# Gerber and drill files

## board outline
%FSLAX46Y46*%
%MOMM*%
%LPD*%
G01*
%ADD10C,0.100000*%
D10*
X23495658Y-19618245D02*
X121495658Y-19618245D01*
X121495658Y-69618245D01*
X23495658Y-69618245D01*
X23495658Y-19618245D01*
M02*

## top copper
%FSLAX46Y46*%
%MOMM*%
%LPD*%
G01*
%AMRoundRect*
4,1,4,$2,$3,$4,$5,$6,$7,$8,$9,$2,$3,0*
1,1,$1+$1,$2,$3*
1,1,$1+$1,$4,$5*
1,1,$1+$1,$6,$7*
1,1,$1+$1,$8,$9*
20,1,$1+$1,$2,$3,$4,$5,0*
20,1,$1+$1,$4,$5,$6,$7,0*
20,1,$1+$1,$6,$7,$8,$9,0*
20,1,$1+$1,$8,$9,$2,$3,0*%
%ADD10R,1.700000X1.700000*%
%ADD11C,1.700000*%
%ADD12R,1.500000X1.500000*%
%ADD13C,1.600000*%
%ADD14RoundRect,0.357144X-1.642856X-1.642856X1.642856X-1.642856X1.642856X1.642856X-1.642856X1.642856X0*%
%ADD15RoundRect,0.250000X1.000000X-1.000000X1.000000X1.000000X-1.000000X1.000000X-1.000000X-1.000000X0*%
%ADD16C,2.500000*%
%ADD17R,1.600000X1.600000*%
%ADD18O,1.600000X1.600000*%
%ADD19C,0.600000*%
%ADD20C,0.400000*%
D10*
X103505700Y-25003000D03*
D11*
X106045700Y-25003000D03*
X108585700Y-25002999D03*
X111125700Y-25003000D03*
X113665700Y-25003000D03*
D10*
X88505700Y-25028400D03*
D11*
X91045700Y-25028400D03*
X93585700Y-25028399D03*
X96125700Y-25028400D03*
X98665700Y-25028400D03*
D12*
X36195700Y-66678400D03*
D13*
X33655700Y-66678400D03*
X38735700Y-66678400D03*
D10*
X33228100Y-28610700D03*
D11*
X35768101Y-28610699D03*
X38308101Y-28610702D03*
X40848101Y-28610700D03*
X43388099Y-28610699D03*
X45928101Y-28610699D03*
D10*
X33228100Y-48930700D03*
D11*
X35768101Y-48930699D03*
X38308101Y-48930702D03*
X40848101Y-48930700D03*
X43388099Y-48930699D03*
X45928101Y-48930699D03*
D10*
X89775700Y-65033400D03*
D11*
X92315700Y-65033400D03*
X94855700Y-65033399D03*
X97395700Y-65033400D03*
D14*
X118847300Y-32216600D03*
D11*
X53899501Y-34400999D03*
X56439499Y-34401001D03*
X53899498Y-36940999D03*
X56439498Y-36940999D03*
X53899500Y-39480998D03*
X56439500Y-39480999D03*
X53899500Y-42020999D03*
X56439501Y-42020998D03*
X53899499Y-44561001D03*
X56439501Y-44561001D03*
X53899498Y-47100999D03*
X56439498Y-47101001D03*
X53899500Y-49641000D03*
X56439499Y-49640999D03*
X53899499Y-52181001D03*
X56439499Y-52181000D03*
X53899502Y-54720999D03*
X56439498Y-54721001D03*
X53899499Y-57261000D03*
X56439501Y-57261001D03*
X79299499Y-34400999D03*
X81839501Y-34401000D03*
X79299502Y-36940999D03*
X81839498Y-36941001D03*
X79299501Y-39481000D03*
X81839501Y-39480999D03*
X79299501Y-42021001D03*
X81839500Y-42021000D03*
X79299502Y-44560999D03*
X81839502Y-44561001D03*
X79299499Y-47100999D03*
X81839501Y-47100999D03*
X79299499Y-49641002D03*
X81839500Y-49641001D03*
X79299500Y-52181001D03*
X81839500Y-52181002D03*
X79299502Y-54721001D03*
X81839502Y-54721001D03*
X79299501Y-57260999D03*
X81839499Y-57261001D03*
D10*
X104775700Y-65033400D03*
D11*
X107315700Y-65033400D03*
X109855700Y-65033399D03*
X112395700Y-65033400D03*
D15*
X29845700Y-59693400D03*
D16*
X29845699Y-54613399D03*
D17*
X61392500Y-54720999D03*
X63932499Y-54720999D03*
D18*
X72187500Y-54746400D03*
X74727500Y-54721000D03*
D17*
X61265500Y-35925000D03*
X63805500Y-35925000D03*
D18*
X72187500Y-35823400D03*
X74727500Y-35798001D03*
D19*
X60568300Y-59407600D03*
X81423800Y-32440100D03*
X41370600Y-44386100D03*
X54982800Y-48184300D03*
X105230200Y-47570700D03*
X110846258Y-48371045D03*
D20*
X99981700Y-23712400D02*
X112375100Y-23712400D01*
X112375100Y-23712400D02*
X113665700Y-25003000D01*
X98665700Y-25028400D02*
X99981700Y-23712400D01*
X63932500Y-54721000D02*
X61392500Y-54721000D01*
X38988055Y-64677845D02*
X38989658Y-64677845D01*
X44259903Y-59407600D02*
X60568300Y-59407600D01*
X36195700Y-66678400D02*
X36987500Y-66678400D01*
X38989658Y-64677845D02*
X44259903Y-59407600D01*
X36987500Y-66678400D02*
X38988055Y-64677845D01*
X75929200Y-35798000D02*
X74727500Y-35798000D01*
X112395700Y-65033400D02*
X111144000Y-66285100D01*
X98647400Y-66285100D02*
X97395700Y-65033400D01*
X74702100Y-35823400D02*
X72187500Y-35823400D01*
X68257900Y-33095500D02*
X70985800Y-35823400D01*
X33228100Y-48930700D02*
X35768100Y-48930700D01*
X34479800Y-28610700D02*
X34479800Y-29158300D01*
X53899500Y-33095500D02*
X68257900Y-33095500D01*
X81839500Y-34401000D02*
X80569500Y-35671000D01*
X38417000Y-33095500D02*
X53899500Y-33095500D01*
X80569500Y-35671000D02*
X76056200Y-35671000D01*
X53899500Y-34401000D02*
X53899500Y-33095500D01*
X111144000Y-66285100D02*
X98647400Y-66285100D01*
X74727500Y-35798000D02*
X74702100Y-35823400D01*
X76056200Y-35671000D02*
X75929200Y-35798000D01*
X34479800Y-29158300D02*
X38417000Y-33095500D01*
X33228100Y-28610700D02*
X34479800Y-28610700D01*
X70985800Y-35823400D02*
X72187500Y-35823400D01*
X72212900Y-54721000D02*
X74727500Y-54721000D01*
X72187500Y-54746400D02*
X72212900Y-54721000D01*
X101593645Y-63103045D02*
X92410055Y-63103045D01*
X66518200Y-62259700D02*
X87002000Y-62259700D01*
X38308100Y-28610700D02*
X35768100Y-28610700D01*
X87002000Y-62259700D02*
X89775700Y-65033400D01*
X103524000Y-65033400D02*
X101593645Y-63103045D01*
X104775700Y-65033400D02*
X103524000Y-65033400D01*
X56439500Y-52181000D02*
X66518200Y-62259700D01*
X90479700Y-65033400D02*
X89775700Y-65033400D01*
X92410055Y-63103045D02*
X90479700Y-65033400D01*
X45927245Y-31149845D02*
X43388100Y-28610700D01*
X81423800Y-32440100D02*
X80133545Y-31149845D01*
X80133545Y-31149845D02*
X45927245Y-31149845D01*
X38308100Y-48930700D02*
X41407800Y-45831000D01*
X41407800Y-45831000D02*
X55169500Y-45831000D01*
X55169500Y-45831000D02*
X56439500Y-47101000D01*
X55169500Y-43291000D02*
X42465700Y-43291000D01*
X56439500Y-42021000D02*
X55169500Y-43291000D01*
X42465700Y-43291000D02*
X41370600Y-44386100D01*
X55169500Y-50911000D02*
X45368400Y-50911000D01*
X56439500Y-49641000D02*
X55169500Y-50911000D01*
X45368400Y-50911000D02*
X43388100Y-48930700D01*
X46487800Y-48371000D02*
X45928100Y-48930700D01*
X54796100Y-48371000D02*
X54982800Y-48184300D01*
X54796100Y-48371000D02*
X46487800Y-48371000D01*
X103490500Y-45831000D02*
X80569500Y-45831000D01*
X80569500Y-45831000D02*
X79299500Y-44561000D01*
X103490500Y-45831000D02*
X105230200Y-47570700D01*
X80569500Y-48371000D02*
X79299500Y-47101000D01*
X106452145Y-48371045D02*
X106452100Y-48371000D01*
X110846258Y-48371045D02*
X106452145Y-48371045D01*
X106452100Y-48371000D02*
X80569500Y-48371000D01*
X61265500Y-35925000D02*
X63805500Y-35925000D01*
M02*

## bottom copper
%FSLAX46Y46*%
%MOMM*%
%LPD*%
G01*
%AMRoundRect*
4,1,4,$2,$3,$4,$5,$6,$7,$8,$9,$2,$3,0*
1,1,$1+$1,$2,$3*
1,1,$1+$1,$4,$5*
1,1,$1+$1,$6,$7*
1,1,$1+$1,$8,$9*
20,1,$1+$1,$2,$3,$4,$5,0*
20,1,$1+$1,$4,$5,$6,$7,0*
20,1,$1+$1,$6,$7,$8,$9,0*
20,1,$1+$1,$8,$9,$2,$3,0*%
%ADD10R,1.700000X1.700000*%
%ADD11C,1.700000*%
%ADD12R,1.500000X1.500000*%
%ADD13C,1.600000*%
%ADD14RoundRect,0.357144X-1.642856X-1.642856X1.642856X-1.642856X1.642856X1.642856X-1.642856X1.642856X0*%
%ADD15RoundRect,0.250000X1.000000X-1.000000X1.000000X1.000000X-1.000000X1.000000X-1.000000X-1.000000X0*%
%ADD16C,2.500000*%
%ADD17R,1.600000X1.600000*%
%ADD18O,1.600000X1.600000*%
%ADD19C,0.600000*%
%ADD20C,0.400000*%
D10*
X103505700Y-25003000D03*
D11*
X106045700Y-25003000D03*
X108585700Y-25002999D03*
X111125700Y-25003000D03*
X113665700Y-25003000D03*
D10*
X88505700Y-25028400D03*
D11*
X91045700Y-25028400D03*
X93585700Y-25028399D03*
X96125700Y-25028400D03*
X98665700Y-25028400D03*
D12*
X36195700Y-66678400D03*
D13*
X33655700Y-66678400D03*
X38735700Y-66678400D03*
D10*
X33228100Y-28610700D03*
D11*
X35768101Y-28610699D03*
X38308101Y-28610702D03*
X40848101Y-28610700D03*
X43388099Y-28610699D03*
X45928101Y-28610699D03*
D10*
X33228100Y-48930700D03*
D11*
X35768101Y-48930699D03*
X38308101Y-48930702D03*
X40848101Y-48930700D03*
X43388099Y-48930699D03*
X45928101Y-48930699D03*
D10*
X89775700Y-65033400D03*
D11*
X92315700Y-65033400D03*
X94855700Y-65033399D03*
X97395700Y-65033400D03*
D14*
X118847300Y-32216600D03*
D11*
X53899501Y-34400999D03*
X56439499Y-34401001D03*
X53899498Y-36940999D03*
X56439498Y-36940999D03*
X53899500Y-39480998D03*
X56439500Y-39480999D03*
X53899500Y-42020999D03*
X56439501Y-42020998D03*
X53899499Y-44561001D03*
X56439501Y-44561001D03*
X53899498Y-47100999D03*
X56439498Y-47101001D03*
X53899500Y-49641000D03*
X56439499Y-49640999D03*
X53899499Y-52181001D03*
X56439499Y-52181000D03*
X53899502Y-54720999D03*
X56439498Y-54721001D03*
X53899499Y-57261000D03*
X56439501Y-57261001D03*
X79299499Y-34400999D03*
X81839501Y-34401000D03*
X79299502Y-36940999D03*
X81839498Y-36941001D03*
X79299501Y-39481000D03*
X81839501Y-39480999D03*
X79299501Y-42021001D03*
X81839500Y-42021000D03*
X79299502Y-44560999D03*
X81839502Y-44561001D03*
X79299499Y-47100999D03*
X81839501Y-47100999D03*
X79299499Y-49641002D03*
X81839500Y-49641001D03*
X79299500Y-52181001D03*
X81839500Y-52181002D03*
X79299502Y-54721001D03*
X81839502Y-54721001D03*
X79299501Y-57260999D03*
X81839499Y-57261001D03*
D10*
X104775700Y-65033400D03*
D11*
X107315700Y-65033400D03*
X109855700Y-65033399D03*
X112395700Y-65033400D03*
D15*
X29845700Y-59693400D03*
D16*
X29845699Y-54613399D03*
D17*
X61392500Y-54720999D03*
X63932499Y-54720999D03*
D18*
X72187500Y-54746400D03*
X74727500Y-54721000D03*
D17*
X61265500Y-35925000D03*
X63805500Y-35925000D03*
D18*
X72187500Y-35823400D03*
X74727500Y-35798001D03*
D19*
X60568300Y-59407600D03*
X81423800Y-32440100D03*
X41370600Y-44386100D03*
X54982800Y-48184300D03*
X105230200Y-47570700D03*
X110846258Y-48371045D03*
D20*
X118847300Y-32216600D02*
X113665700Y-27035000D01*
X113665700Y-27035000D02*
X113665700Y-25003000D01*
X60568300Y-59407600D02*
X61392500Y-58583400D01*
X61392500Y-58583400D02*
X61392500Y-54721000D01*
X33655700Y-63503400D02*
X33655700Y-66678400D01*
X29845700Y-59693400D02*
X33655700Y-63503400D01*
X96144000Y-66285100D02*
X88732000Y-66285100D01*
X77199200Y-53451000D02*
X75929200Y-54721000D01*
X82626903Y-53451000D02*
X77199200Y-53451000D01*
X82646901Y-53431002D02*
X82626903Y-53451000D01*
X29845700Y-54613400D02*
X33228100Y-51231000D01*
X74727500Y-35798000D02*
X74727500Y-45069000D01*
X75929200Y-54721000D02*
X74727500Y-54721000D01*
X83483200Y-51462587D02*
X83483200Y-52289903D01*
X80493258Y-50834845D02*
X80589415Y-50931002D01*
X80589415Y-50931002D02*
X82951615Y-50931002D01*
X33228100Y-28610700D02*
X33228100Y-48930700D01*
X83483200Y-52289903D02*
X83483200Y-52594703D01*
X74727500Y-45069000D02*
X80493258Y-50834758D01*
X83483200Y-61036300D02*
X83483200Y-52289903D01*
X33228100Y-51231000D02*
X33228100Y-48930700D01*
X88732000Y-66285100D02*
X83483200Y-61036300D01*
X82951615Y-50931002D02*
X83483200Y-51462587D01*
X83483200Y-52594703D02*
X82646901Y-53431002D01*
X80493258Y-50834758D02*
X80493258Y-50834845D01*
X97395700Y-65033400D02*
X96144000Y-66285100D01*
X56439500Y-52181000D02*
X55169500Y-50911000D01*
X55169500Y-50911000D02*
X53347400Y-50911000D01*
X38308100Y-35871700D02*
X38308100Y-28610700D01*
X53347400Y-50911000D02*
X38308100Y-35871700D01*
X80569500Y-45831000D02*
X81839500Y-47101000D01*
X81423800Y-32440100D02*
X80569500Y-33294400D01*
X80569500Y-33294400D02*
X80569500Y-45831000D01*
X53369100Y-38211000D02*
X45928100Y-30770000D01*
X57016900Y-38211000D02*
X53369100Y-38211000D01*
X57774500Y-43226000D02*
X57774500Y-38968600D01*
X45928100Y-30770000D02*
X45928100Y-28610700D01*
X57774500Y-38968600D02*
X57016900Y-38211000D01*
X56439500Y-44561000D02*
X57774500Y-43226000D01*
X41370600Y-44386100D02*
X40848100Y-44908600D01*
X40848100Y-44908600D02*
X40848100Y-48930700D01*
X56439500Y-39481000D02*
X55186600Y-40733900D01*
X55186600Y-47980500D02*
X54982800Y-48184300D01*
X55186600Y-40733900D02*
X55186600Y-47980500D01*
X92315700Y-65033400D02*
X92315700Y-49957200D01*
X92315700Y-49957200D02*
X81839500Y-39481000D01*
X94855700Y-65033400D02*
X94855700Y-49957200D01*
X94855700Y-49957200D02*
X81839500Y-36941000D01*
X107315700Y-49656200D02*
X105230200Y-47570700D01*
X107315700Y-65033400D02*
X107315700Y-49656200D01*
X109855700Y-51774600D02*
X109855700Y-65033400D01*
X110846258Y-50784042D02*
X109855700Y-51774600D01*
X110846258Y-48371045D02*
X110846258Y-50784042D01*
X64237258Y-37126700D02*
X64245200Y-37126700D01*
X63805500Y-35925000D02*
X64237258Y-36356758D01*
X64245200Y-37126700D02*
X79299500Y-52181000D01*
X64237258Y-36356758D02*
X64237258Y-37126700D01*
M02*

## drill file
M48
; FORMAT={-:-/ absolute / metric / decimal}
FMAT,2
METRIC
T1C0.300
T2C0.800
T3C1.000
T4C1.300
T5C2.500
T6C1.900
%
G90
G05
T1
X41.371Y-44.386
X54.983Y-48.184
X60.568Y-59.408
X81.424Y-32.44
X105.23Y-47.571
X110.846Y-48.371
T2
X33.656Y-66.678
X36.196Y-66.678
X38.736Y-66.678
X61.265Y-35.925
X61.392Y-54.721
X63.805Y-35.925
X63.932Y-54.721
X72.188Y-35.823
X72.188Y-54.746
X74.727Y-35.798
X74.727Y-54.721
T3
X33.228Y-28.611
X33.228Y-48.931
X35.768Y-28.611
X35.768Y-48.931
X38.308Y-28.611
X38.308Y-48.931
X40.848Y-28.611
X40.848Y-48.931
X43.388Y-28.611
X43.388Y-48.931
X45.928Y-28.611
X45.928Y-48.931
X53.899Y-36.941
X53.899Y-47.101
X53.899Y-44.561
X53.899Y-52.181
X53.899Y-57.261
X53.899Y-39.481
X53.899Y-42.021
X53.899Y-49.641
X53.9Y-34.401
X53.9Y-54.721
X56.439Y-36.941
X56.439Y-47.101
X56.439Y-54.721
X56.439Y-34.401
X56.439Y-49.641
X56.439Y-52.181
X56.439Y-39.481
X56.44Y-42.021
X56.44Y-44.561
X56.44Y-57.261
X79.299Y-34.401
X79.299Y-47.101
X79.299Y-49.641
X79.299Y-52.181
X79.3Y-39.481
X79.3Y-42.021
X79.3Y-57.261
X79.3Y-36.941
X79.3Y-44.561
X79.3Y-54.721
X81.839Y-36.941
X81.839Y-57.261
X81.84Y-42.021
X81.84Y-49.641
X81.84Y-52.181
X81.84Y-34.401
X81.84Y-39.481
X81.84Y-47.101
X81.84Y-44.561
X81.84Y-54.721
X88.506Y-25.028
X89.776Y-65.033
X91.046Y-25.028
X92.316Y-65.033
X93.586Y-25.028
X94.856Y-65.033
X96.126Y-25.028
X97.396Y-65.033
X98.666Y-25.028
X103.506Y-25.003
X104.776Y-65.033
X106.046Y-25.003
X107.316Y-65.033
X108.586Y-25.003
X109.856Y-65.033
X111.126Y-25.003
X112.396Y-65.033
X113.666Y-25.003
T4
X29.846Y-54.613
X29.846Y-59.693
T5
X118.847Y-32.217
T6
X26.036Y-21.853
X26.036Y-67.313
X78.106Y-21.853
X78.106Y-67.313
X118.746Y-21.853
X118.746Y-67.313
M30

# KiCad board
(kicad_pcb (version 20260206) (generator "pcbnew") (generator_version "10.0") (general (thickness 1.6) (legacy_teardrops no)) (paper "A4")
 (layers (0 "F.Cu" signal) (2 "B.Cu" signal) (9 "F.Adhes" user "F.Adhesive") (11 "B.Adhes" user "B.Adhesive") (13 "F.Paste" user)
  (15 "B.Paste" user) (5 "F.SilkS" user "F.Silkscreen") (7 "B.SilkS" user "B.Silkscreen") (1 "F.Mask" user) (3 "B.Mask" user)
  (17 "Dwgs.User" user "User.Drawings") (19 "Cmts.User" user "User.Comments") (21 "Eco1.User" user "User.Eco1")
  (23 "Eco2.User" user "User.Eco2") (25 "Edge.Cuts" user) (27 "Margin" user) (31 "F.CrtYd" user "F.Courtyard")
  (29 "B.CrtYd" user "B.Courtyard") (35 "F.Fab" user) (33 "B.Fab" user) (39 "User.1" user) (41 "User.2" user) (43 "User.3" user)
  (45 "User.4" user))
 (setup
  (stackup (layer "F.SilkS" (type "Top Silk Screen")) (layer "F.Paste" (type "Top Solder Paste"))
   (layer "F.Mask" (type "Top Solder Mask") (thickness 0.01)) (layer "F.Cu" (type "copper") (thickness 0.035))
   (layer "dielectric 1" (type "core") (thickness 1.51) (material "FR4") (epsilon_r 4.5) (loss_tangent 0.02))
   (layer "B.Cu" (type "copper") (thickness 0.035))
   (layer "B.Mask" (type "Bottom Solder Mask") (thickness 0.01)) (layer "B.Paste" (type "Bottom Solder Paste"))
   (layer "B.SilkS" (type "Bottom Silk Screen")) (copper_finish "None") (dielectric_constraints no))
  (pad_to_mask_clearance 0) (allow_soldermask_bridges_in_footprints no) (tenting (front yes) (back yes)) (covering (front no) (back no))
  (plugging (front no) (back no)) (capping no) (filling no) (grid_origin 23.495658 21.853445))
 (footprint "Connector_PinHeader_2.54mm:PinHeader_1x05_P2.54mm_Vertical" (layer "F.Cu") (at 103.5057 25.003 90)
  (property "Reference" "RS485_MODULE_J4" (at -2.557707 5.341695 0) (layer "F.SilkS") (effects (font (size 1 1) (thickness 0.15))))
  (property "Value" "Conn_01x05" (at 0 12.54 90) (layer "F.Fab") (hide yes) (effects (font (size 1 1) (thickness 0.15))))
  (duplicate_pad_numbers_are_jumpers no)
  (pad "1" thru_hole rect (at 0 0 90) (size 1.7 1.7) (drill 1) (layers "*.Cu" "*.Mask") (remove_unused_layers no)
   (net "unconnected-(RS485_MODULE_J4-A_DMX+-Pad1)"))
  (pad "2" thru_hole circle (at 0 2.54 90) (size 1.7 1.7) (drill 1) (layers "*.Cu" "*.Mask") (remove_unused_layers no)
   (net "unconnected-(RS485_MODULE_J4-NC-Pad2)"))
  (pad "3" thru_hole circle (at 0.000001 5.08 90) (size 1.7 1.7) (drill 1) (layers "*.Cu" "*.Mask") (remove_unused_layers no)
   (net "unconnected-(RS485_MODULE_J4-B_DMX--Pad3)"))
  (pad "4" thru_hole circle (at 0 7.62 90) (size 1.7 1.7) (drill 1) (layers "*.Cu" "*.Mask") (remove_unused_layers no)
   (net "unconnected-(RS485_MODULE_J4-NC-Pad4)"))
  (pad "5" thru_hole circle (at 0 10.16 90) (size 1.7 1.7) (drill 1) (layers "*.Cu" "*.Mask") (remove_unused_layers no) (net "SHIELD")))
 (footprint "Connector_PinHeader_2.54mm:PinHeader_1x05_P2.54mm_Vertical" (layer "F.Cu") (at 88.5057 25.0284 90)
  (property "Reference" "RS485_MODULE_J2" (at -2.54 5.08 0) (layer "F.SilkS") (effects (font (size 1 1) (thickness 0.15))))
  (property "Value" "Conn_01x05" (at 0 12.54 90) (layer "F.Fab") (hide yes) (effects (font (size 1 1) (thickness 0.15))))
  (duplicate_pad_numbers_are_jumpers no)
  (pad "1" thru_hole rect (at 0 0 90) (size 1.7 1.7) (drill 1) (layers "*.Cu" "*.Mask") (remove_unused_layers no)
   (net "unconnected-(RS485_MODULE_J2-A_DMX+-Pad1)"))
  (pad "2" thru_hole circle (at 0 2.54 90) (size 1.7 1.7) (drill 1) (layers "*.Cu" "*.Mask") (remove_unused_layers no)
   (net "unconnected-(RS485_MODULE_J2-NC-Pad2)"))
  (pad "3" thru_hole circle (at 0.000001 5.08 90) (size 1.7 1.7) (drill 1) (layers "*.Cu" "*.Mask") (remove_unused_layers no)
   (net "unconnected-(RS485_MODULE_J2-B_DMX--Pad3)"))
  (pad "4" thru_hole circle (at 0 7.62 90) (size 1.7 1.7) (drill 1) (layers "*.Cu" "*.Mask") (remove_unused_layers no)
   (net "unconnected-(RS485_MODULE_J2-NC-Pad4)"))
  (pad "5" thru_hole circle (at 0 10.16 90) (size 1.7 1.7) (drill 1) (layers "*.Cu" "*.Mask") (remove_unused_layers no) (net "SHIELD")))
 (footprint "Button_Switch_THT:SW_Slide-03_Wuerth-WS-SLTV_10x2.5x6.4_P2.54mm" (layer "F.Cu") (at 36.1957 66.6784)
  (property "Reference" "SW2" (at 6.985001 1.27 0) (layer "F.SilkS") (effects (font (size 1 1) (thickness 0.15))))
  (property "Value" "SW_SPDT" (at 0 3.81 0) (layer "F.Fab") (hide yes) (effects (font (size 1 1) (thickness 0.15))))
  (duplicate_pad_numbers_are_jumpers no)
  (pad "1" thru_hole rect (at 0 0) (size 1.5 1.5) (drill 0.8) (layers "*.Cu" "*.Mask") (remove_unused_layers no)
   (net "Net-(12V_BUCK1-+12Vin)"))
  (pad "2" thru_hole circle (at -2.54 0) (size 1.6 1.6) (drill 0.8) (layers "*.Cu" "*.Mask") (remove_unused_layers no) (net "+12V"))
  (pad "3" thru_hole circle (at 2.54 0) (size 1.6 1.6) (drill 0.8) (layers "*.Cu" "*.Mask") (remove_unused_layers no)
   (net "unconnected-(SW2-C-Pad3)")))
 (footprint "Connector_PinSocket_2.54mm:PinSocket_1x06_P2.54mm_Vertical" (layer "F.Cu") (at 33.2281 28.6107 90)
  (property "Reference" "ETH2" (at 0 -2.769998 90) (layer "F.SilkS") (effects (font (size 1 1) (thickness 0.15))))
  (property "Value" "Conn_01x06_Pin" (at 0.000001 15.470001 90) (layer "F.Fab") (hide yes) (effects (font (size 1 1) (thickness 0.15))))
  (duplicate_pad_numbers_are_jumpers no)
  (pad "1" thru_hole rect (at 0 0 90) (size 1.7 1.7) (drill 1) (layers "*.Cu" "*.Mask") (remove_unused_layers yes) (keep_end_layers yes)
   (zone_layer_connections) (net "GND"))
  (pad "2" thru_hole circle (at 0.000001 2.540001 90) (size 1.7 1.7) (drill 1) (layers "*.Cu" "*.Mask") (remove_unused_layers yes)
   (keep_end_layers yes) (zone_layer_connections) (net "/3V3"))
  (pad "3" thru_hole circle (at -0.000002 5.080001 90) (size 1.7 1.7) (drill 1) (layers "*.Cu" "*.Mask") (remove_unused_layers yes)
   (keep_end_layers yes) (zone_layer_connections) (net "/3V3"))
  (pad "4" thru_hole circle (at 0 7.620001 90) (size 1.7 1.7) (drill 1) (layers "*.Cu" "*.Mask") (remove_unused_layers yes)
   (keep_end_layers yes) (zone_layer_connections) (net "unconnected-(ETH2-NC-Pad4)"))
  (pad "5" thru_hole circle (at 0.000001 10.159999 90) (size 1.7 1.7) (drill 1) (layers "*.Cu" "*.Mask") (remove_unused_layers yes)
   (keep_end_layers yes) (zone_layer_connections) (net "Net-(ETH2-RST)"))
  (pad "6" thru_hole circle (at 0.000001 12.700001 90) (size 1.7 1.7) (drill 1) (layers "*.Cu" "*.Mask") (remove_unused_layers yes)
   (keep_end_layers yes) (zone_layer_connections) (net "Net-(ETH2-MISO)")))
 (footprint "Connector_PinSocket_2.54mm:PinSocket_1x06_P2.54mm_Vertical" (layer "F.Cu") (at 33.2281 48.9307 90)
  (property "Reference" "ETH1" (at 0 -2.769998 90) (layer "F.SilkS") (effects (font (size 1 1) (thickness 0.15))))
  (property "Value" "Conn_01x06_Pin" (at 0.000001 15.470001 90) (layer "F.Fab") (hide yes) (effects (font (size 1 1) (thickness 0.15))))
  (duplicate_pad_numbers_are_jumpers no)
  (pad "1" thru_hole rect (at 0 0 90) (size 1.7 1.7) (drill 1) (layers "*.Cu" "*.Mask") (remove_unused_layers yes) (keep_end_layers yes)
   (zone_layer_connections) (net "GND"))
  (pad "2" thru_hole circle (at 0.000001 2.540001 90) (size 1.7 1.7) (drill 1) (layers "*.Cu" "*.Mask") (remove_unused_layers yes)
   (keep_end_layers yes) (zone_layer_connections) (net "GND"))
  (pad "3" thru_hole circle (at -0.000002 5.080001 90) (size 1.7 1.7) (drill 1) (layers "*.Cu" "*.Mask") (remove_unused_layers yes)
   (keep_end_layers yes) (zone_layer_connections) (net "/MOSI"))
  (pad "4" thru_hole circle (at 0 7.620001 90) (size 1.7 1.7) (drill 1) (layers "*.Cu" "*.Mask") (remove_unused_layers yes)
   (keep_end_layers yes) (zone_layer_connections) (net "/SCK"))
  (pad "5" thru_hole circle (at 0.000001 10.159999 90) (size 1.7 1.7) (drill 1) (layers "*.Cu" "*.Mask") (remove_unused_layers yes)
   (keep_end_layers yes) (zone_layer_connections) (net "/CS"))
  (pad "6" thru_hole circle (at 0.000001 12.700001 90) (size 1.7 1.7) (drill 1) (layers "*.Cu" "*.Mask") (remove_unused_layers yes)
   (keep_end_layers yes) (zone_layer_connections) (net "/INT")))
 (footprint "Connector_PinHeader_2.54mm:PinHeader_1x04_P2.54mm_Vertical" (layer "F.Cu") (at 89.7757 65.0334 90)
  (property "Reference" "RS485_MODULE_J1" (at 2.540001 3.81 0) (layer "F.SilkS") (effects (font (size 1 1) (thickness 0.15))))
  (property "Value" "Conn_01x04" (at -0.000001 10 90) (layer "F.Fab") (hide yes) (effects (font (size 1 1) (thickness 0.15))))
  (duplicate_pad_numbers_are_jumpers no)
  (pad "1" thru_hole rect (at 0 0 90) (size 1.7 1.7) (drill 1) (layers "*.Cu" "*.Mask") (remove_unused_layers no) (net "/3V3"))
  (pad "2" thru_hole circle (at 0 2.54 90) (size 1.7 1.7) (drill 1) (layers "*.Cu" "*.Mask") (remove_unused_layers no)
   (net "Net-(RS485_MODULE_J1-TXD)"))
  (pad "3" thru_hole circle (at 0.000001 5.08 90) (size 1.7 1.7) (drill 1) (layers "*.Cu" "*.Mask") (remove_unused_layers no)
   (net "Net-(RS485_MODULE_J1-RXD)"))
  (pad "4" thru_hole circle (at 0 7.62 90) (size 1.7 1.7) (drill 1) (layers "*.Cu" "*.Mask") (remove_unused_layers no) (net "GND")))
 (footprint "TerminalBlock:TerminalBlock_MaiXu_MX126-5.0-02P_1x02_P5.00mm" (layer "F.Cu") (at 118.8473 32.2166)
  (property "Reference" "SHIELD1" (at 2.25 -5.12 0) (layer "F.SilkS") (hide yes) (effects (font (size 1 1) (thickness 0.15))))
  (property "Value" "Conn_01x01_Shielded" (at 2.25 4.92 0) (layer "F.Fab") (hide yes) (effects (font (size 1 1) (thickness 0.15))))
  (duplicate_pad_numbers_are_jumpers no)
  (pad "1" thru_hole roundrect (at 0 0) (size 4 4) (drill 2.5) (layers "*.Cu" "*.Mask") (remove_unused_layers no)
   (roundrect_rratio 0.089286) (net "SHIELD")))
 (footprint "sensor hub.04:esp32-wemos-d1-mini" (layer "F.Cu") (at 67.8695 45.831)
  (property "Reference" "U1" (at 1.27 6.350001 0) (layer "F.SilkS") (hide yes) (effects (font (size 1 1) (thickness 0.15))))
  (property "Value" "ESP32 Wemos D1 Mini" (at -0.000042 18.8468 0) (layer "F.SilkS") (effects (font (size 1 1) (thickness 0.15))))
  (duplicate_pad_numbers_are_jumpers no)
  (pad "1" thru_hole circle (at -13.969999 -11.430001) (size 1.7 1.7) (drill 1) (layers "*.Cu" "*.Mask") (remove_unused_layers yes)
   (keep_end_layers yes) (zone_layer_connections) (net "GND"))
  (pad "2" thru_hole circle (at -11.430001 -11.429999) (size 1.7 1.7) (drill 1) (layers "*.Cu" "*.Mask") (remove_unused_layers yes)
   (keep_end_layers yes) (zone_layer_connections) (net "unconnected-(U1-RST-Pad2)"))
  (pad "3" thru_hole circle (at -13.970002 -8.890001) (size 1.7 1.7) (drill 1) (layers "*.Cu" "*.Mask") (remove_unused_layers yes)
   (keep_end_layers yes) (zone_layer_connections) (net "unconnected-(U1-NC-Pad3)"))
  (pad "4" thru_hole circle (at -11.430002 -8.890001) (size 1.7 1.7) (drill 1) (layers "*.Cu" "*.Mask") (remove_unused_layers yes)
   (keep_end_layers yes) (zone_layer_connections) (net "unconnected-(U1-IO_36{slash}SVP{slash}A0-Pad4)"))
  (pad "5" thru_hole circle (at -13.97 -6.350002) (size 1.7 1.7) (drill 1) (layers "*.Cu" "*.Mask") (remove_unused_layers yes)
   (keep_end_layers yes) (zone_layer_connections) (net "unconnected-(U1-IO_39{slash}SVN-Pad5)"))
  (pad "6" thru_hole circle (at -11.43 -6.350001) (size 1.7 1.7) (drill 1) (layers "*.Cu" "*.Mask") (remove_unused_layers yes)
   (keep_end_layers yes) (zone_layer_connections) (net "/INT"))
  (pad "7" thru_hole circle (at -13.97 -3.810001) (size 1.7 1.7) (drill 1) (layers "*.Cu" "*.Mask") (remove_unused_layers yes)
   (keep_end_layers yes) (zone_layer_connections) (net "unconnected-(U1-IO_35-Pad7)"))
  (pad "8" thru_hole circle (at -11.429999 -3.810002) (size 1.7 1.7) (drill 1) (layers "*.Cu" "*.Mask") (remove_unused_layers yes)
   (keep_end_layers yes) (zone_layer_connections) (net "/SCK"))
  (pad "9" thru_hole circle (at -13.970001 -1.269999) (size 1.7 1.7) (drill 1) (layers "*.Cu" "*.Mask") (remove_unused_layers yes)
   (keep_end_layers yes) (zone_layer_connections) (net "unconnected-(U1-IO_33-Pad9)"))
  (pad "10" thru_hole circle (at -11.429999 -1.269999) (size 1.7 1.7) (drill 1) (layers "*.Cu" "*.Mask") (remove_unused_layers yes)
   (keep_end_layers yes) (zone_layer_connections) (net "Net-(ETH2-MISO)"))
  (pad "11" thru_hole circle (at -13.970002 1.269999) (size 1.7 1.7) (drill 1) (layers "*.Cu" "*.Mask") (remove_unused_layers yes)
   (keep_end_layers yes) (zone_layer_connections) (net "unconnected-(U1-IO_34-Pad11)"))
  (pad "12" thru_hole circle (at -11.430002 1.270001) (size 1.7 1.7) (drill 1) (layers "*.Cu" "*.Mask") (remove_unused_layers yes)
   (keep_end_layers yes) (zone_layer_connections) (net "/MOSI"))
  (pad "13" thru_hole circle (at -13.97 3.81) (size 1.7 1.7) (drill 1) (layers "*.Cu" "*.Mask") (remove_unused_layers yes)
   (keep_end_layers yes) (zone_layer_connections) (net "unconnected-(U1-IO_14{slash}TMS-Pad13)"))
  (pad "14" thru_hole circle (at -11.430001 3.809999) (size 1.7 1.7) (drill 1) (layers "*.Cu" "*.Mask") (remove_unused_layers yes)
   (keep_end_layers yes) (zone_layer_connections) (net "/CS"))
  (pad "15" thru_hole circle (at -13.970001 6.350001) (size 1.7 1.7) (drill 1) (layers "*.Cu" "*.Mask") (remove_unused_layers yes)
   (keep_end_layers yes) (zone_layer_connections) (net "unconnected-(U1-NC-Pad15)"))
  (pad "16" thru_hole circle (at -11.430001 6.35) (size 1.7 1.7) (drill 1) (layers "*.Cu" "*.Mask") (remove_unused_layers yes)
   (keep_end_layers yes) (zone_layer_connections) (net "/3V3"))
  (pad "17" thru_hole circle (at -13.969998 8.889999) (size 1.7 1.7) (drill 1) (layers "*.Cu" "*.Mask") (remove_unused_layers yes)
   (keep_end_layers yes) (zone_layer_connections) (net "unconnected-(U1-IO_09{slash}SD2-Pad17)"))
  (pad "18" thru_hole circle (at -11.430002 8.890001) (size 1.7 1.7) (drill 1) (layers "*.Cu" "*.Mask") (remove_unused_layers yes)
   (keep_end_layers yes) (zone_layer_connections) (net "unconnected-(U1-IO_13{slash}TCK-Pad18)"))
  (pad "19" thru_hole circle (at -13.970001 11.43) (size 1.7 1.7) (drill 1) (layers "*.Cu" "*.Mask") (remove_unused_layers yes)
   (keep_end_layers yes) (zone_layer_connections) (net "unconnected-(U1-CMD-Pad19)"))
  (pad "20" thru_hole circle (at -11.429999 11.430001) (size 1.7 1.7) (drill 1) (layers "*.Cu" "*.Mask") (remove_unused_layers yes)
   (keep_end_layers yes) (zone_layer_connections) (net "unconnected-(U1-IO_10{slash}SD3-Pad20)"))
  (pad "21" thru_hole circle (at 11.429999 -11.430001) (size 1.7 1.7) (drill 1) (layers "*.Cu" "*.Mask") (remove_unused_layers yes)
   (keep_end_layers yes) (zone_layer_connections) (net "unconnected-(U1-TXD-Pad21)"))
  (pad "22" thru_hole circle (at 13.970001 -11.43) (size 1.7 1.7) (drill 1) (layers "*.Cu" "*.Mask") (remove_unused_layers yes)
   (keep_end_layers yes) (zone_layer_connections) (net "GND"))
  (pad "23" thru_hole circle (at 11.430002 -8.890001) (size 1.7 1.7) (drill 1) (layers "*.Cu" "*.Mask") (remove_unused_layers yes)
   (keep_end_layers yes) (zone_layer_connections) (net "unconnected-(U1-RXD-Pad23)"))
  (pad "24" thru_hole circle (at 13.969998 -8.889999) (size 1.7 1.7) (drill 1) (layers "*.Cu" "*.Mask") (remove_unused_layers yes)
   (keep_end_layers yes) (zone_layer_connections) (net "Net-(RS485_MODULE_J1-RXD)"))
  (pad "25" thru_hole circle (at 11.430001 -6.35) (size 1.7 1.7) (drill 1) (layers "*.Cu" "*.Mask") (remove_unused_layers yes)
   (keep_end_layers yes) (zone_layer_connections) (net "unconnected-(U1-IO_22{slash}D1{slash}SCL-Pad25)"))
  (pad "26" thru_hole circle (at 13.970001 -6.350001) (size 1.7 1.7) (drill 1) (layers "*.Cu" "*.Mask") (remove_unused_layers yes)
   (keep_end_layers yes) (zone_layer_connections) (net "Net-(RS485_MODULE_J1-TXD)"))
  (pad "27" thru_hole circle (at 11.430001 -3.809999) (size 1.7 1.7) (drill 1) (layers "*.Cu" "*.Mask") (remove_unused_layers yes)
   (keep_end_layers yes) (zone_layer_connections) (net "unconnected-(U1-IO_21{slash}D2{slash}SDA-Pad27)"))
  (pad "28" thru_hole circle (at 13.97 -3.81) (size 1.7 1.7) (drill 1) (layers "*.Cu" "*.Mask") (remove_unused_layers yes)
   (keep_end_layers yes) (zone_layer_connections) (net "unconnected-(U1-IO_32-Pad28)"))
  (pad "29" thru_hole circle (at 11.430002 -1.270001) (size 1.7 1.7) (drill 1) (layers "*.Cu" "*.Mask") (remove_unused_layers yes)
   (keep_end_layers yes) (zone_layer_connections) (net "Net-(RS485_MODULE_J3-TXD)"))
  (pad "30" thru_hole circle (at 13.970002 -1.269999) (size 1.7 1.7) (drill 1) (layers "*.Cu" "*.Mask") (remove_unused_layers yes)
   (keep_end_layers yes) (zone_layer_connections) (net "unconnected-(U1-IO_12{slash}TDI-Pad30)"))
  (pad "31" thru_hole circle (at 11.429999 1.269999) (size 1.7 1.7) (drill 1) (layers "*.Cu" "*.Mask") (remove_unused_layers yes)
   (keep_end_layers yes) (zone_layer_connections) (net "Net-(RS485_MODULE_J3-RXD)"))
  (pad "32" thru_hole circle (at 13.970001 1.269999) (size 1.7 1.7) (drill 1) (layers "*.Cu" "*.Mask") (remove_unused_layers yes)
   (keep_end_layers yes) (zone_layer_connections) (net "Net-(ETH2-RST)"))
  (pad "33" thru_hole circle (at 11.429999 3.810002) (size 1.7 1.7) (drill 1) (layers "*.Cu" "*.Mask") (remove_unused_layers yes)
   (keep_end_layers yes) (zone_layer_connections) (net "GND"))
  (pad "34" thru_hole circle (at 13.97 3.810001) (size 1.7 1.7) (drill 1) (layers "*.Cu" "*.Mask") (remove_unused_layers yes)
   (keep_end_layers yes) (zone_layer_connections) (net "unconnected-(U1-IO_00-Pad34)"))
  (pad "35" thru_hole circle (at 11.43 6.350001) (size 1.7 1.7) (drill 1) (layers "*.Cu" "*.Mask") (remove_unused_layers yes)
   (keep_end_layers yes) (zone_layer_connections) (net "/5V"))
  (pad "36" thru_hole circle (at 13.97 6.350002) (size 1.7 1.7) (drill 1) (layers "*.Cu" "*.Mask") (remove_unused_layers yes)
   (keep_end_layers yes) (zone_layer_connections) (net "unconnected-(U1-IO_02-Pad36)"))
  (pad "37" thru_hole circle (at 11.430002 8.890001) (size 1.7 1.7) (drill 1) (layers "*.Cu" "*.Mask") (remove_unused_layers yes)
   (keep_end_layers yes) (zone_layer_connections) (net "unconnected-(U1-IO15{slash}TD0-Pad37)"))
  (pad "38" thru_hole circle (at 13.970002 8.890001) (size 1.7 1.7) (drill 1) (layers "*.Cu" "*.Mask") (remove_unused_layers yes)
   (keep_end_layers yes) (zone_layer_connections) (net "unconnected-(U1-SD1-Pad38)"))
  (pad "39" thru_hole circle (at 11.430001 11.429999) (size 1.7 1.7) (drill 1) (layers "*.Cu" "*.Mask") (remove_unused_layers yes)
   (keep_end_layers yes) (zone_layer_connections) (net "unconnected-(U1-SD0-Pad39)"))
  (pad "40" thru_hole circle (at 13.969999 11.430001) (size 1.7 1.7) (drill 1) (layers "*.Cu" "*.Mask") (remove_unused_layers yes)
   (keep_end_layers yes) (zone_layer_connections) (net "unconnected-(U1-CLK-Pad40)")))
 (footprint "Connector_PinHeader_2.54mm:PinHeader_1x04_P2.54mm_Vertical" (layer "F.Cu") (at 104.7757 65.0334 90)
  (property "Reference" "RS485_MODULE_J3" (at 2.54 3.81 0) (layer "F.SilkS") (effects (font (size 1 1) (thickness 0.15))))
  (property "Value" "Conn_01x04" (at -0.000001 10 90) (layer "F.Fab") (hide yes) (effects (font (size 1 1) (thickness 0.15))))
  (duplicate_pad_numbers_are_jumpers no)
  (pad "1" thru_hole rect (at 0 0 90) (size 1.7 1.7) (drill 1) (layers "*.Cu" "*.Mask") (remove_unused_layers no) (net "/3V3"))
  (pad "2" thru_hole circle (at 0 2.54 90) (size 1.7 1.7) (drill 1) (layers "*.Cu" "*.Mask") (remove_unused_layers no)
   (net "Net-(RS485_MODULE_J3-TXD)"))
  (pad "3" thru_hole circle (at 0.000001 5.08 90) (size 1.7 1.7) (drill 1) (layers "*.Cu" "*.Mask") (remove_unused_layers no)
   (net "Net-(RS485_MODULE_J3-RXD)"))
  (pad "4" thru_hole circle (at 0 7.62 90) (size 1.7 1.7) (drill 1) (layers "*.Cu" "*.Mask") (remove_unused_layers no) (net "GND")))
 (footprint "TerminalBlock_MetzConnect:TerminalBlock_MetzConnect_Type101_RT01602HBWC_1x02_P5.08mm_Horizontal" (layer "F.Cu")
  (at 29.8457 59.6934 90)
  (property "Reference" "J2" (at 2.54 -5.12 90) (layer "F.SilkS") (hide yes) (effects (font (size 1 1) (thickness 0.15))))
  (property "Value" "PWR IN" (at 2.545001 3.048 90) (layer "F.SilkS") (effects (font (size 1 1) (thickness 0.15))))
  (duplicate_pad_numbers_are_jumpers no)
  (pad "1" thru_hole roundrect (at 0 0 90) (size 2.5 2.5) (drill 1.3) (layers "*.Cu" "*.Mask") (remove_unused_layers no)
   (roundrect_rratio 0.1) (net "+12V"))
  (pad "2" thru_hole circle (at 5.080001 -0.000001 90) (size 2.5 2.5) (drill 1.3) (layers "*.Cu" "*.Mask") (remove_unused_layers no)
   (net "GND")))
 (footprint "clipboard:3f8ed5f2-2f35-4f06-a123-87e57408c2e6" (layer "B.Cu") (at 118.745658 67.313445 180)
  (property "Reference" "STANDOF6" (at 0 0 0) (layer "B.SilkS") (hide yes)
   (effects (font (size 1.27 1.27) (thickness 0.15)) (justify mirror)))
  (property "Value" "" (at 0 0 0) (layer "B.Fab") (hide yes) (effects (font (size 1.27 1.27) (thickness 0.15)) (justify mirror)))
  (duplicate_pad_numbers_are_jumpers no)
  (pad "" np_thru_hole roundrect (at 0 0 180) (size 4 4) (drill 1.9) (layers "*.Mask") (roundrect_rratio 0) (chamfer_ratio 0.3)
   (chamfer top_left top_right bottom_left bottom_right)))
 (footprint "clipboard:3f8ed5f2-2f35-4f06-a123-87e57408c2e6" (layer "B.Cu") (at 118.745658 21.853445 180)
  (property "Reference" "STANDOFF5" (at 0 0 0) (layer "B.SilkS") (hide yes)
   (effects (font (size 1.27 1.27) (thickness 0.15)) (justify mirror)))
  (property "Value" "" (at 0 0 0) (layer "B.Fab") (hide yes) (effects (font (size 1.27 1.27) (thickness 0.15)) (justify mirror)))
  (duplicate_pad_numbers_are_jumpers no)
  (pad "" np_thru_hole roundrect (at 0 0 180) (size 4 4) (drill 1.9) (layers "*.Mask") (roundrect_rratio 0) (chamfer_ratio 0.3)
   (chamfer top_left top_right bottom_left bottom_right)))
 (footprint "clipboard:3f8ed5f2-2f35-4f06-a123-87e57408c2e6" (layer "B.Cu") (at 78.105658 21.853445 180)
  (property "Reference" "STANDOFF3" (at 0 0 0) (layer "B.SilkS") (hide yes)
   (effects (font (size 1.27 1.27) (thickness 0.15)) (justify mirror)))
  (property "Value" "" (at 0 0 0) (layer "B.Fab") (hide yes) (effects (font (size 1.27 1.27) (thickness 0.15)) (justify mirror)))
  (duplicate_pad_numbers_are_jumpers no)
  (pad "" np_thru_hole roundrect (at 0 0 180) (size 4 4) (drill 1.9) (layers "*.Mask") (roundrect_rratio 0) (chamfer_ratio 0.3)
   (chamfer top_left top_right bottom_left bottom_right)))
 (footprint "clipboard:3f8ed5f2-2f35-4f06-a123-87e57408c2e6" (layer "B.Cu") (at 26.035658 21.853445 180)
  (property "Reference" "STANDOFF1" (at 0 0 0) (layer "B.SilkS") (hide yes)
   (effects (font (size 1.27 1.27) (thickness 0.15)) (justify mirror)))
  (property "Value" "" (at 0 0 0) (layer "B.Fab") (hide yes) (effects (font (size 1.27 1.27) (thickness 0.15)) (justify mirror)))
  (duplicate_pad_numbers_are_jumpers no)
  (pad "" np_thru_hole roundrect (at 0 0 180) (size 4 4) (drill 1.9) (layers "*.Mask") (roundrect_rratio 0) (chamfer_ratio 0.3)
   (chamfer top_left top_right bottom_left bottom_right)))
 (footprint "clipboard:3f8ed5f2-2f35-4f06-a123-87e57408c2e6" (layer "B.Cu") (at 26.035658 67.313445 180)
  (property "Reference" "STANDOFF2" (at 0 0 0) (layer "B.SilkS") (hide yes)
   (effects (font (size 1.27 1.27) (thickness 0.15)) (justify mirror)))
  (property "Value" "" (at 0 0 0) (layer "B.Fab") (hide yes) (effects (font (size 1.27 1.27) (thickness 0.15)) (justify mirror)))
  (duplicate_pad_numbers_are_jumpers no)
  (pad "" np_thru_hole roundrect (at 0 0 180) (size 4 4) (drill 1.9) (layers "*.Mask") (roundrect_rratio 0) (chamfer_ratio 0.3)
   (chamfer top_left top_right bottom_left bottom_right)))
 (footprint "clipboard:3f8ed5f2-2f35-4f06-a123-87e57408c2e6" (layer "B.Cu") (at 78.105658 67.313445 180)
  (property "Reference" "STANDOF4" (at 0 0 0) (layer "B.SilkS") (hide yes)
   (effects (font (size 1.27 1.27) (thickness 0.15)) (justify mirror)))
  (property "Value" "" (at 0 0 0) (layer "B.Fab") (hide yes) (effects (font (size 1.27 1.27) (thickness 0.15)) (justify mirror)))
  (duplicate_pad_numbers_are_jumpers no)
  (pad "" np_thru_hole roundrect (at 0 0 180) (size 4 4) (drill 1.9) (layers "*.Mask") (roundrect_rratio 0) (chamfer_ratio 0.3)
   (chamfer top_left top_right bottom_left bottom_right)))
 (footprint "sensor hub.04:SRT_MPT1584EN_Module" (layer "B.Cu") (at 68.5045 44.561 90)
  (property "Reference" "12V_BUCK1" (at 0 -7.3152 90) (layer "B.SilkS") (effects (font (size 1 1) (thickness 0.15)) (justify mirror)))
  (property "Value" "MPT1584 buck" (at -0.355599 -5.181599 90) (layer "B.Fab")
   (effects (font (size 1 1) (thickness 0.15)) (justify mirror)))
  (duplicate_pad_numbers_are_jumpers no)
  (pad "1" thru_hole rect (at -10.159999 -7.112) (size 1.6 1.6) (drill 0.8) (layers "*.Cu" "F.Mask") (remove_unused_layers no)
   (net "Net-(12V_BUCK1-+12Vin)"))
  (pad "1" thru_hole rect (at -10.159999 -4.572001) (size 1.6 1.6) (drill 0.8) (layers "*.Cu" "F.Mask") (remove_unused_layers no)
   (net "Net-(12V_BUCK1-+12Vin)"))
  (pad "2" thru_hole oval (at -10.1854 3.683) (size 1.6 1.6) (drill 0.8) (layers "*.Cu" "F.Mask") (remove_unused_layers no) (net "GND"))
  (pad "2" thru_hole oval (at -10.16 6.223) (size 1.6 1.6) (drill 0.8) (layers "*.Cu" "F.Mask") (remove_unused_layers no) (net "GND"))
  (pad "3" thru_hole rect (at 8.636 -7.239) (size 1.6 1.6) (drill 0.8) (layers "*.Cu" "F.Mask") (remove_unused_layers no) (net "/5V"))
  (pad "3" thru_hole rect (at 8.636 -4.699) (size 1.6 1.6) (drill 0.8) (layers "*.Cu" "F.Mask") (remove_unused_layers no) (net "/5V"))
  (pad "4" thru_hole oval (at 8.7376 3.683) (size 1.6 1.6) (drill 0.8) (layers "*.Cu" "F.Mask") (remove_unused_layers no) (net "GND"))
  (pad "4" thru_hole oval (at 8.762999 6.223) (size 1.6 1.6) (drill 0.8) (layers "*.Cu" "F.Mask") (remove_unused_layers no) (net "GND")))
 (gr_rect (start 23.495658 19.618245) (end 121.495658 69.618245) (stroke (width 0.1) (type solid)) (fill no) (layer "Edge.Cuts"))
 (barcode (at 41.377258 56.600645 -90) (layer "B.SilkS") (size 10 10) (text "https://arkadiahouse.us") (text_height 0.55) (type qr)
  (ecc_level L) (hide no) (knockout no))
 (segment (start 99.9817 23.7124) (end 112.3751 23.7124) (width 0.4) (layer "F.Cu") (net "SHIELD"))
 (segment (start 112.3751 23.7124) (end 113.6657 25.003) (width 0.4) (layer "F.Cu") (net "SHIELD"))
 (segment (start 98.6657 25.0284) (end 99.9817 23.7124) (width 0.4) (layer "F.Cu") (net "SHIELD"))
 (segment (start 118.8473 32.2166) (end 113.6657 27.035) (width 0.4) (layer "B.Cu") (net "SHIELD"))
 (segment (start 113.6657 27.035) (end 113.6657 25.003) (width 0.4) (layer "B.Cu") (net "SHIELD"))
 (segment (start 63.9325 54.721) (end 61.3925 54.721) (width 0.4) (layer "F.Cu") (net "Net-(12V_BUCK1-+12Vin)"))
 (segment (start 38.988055 64.677845) (end 38.989658 64.677845) (width 0.4) (layer "F.Cu") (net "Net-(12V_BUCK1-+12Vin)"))
 (segment (start 44.259903 59.4076) (end 60.5683 59.4076) (width 0.4) (layer "F.Cu") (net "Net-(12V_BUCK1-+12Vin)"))
 (segment (start 36.1957 66.6784) (end 36.9875 66.6784) (width 0.4) (layer "F.Cu") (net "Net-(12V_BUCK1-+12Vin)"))
 (segment (start 38.989658 64.677845) (end 44.259903 59.4076) (width 0.4) (layer "F.Cu") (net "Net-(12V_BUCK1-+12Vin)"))
 (segment (start 36.9875 66.6784) (end 38.988055 64.677845) (width 0.4) (layer "F.Cu") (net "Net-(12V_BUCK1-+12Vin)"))
 (via (at 60.5683 59.4076) (size 0.6) (drill 0.3) (layers "F.Cu" "B.Cu") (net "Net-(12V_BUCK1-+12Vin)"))
 (segment (start 60.5683 59.4076) (end 61.3925 58.5834) (width 0.4) (layer "B.Cu") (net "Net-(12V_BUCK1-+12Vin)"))
 (segment (start 61.3925 58.5834) (end 61.3925 54.721) (width 0.4) (layer "B.Cu") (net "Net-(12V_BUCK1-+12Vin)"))
 (segment (start 33.6557 63.5034) (end 33.6557 66.6784) (width 0.4) (layer "B.Cu") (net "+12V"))
 (segment (start 29.8457 59.6934) (end 33.6557 63.5034) (width 0.4) (layer "B.Cu") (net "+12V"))
 (segment (start 75.9292 35.798) (end 74.7275 35.798) (width 0.4) (layer "F.Cu") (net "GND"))
 (segment (start 112.3957 65.0334) (end 111.144 66.2851) (width 0.4) (layer "F.Cu") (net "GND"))
 (segment (start 98.6474 66.2851) (end 97.3957 65.0334) (width 0.4) (layer "F.Cu") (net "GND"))
 (segment (start 74.7021 35.8234) (end 72.1875 35.8234) (width 0.4) (layer "F.Cu") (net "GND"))
 (segment (start 68.2579 33.0955) (end 70.9858 35.8234) (width 0.4) (layer "F.Cu") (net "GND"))
 (segment (start 33.2281 48.9307) (end 35.7681 48.9307) (width 0.4) (layer "F.Cu") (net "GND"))
 (segment (start 34.4798 28.6107) (end 34.4798 29.1583) (width 0.4) (layer "F.Cu") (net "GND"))
 (segment (start 53.8995 33.0955) (end 68.2579 33.0955) (width 0.4) (layer "F.Cu") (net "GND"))
 (segment (start 81.8395 34.401) (end 80.5695 35.671) (width 0.4) (layer "F.Cu") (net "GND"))
 (segment (start 38.417 33.0955) (end 53.8995 33.0955) (width 0.4) (layer "F.Cu") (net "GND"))
 (segment (start 80.5695 35.671) (end 76.0562 35.671) (width 0.4) (layer "F.Cu") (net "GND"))
 (segment (start 53.8995 34.401) (end 53.8995 33.0955) (width 0.4) (layer "F.Cu") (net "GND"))
 (segment (start 111.144 66.2851) (end 98.6474 66.2851) (width 0.4) (layer "F.Cu") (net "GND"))
 (segment (start 74.7275 35.798) (end 74.7021 35.8234) (width 0.4) (layer "F.Cu") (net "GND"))
 (segment (start 76.0562 35.671) (end 75.9292 35.798) (width 0.4) (layer "F.Cu") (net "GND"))
 (segment (start 34.4798 29.1583) (end 38.417 33.0955) (width 0.4) (layer "F.Cu") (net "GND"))
 (segment (start 33.2281 28.6107) (end 34.4798 28.6107) (width 0.4) (layer "F.Cu") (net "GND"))
 (segment (start 70.9858 35.8234) (end 72.1875 35.8234) (width 0.4) (layer "F.Cu") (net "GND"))
 (segment (start 72.2129 54.721) (end 74.7275 54.721) (width 0.4) (layer "F.Cu") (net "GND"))
 (segment (start 72.1875 54.7464) (end 72.2129 54.721) (width 0.4) (layer "F.Cu") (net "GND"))
 (segment (start 96.144 66.2851) (end 88.732 66.2851) (width 0.4) (layer "B.Cu") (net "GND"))
 (segment (start 77.1992 53.451) (end 75.9292 54.721) (width 0.4) (layer "B.Cu") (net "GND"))
 (segment (start 82.626903 53.451) (end 77.1992 53.451) (width 0.4) (layer "B.Cu") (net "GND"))
 (segment (start 82.646901 53.431002) (end 82.626903 53.451) (width 0.4) (layer "B.Cu") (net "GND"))
 (segment (start 29.8457 54.6134) (end 33.2281 51.231) (width 0.4) (layer "B.Cu") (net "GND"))
 (segment (start 74.7275 35.798) (end 74.7275 45.069) (width 0.4) (layer "B.Cu") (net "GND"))
 (segment (start 75.9292 54.721) (end 74.7275 54.721) (width 0.4) (layer "B.Cu") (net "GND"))
 (segment (start 83.4832 51.462587) (end 83.4832 52.289903) (width 0.4) (layer "B.Cu") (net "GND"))
 (segment (start 80.493258 50.834845) (end 80.589415 50.931002) (width 0.4) (layer "B.Cu") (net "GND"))
 (segment (start 80.589415 50.931002) (end 82.951615 50.931002) (width 0.4) (layer "B.Cu") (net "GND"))
 (segment (start 33.2281 28.6107) (end 33.2281 48.9307) (width 0.4) (layer "B.Cu") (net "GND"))
 (segment (start 83.4832 52.289903) (end 83.4832 52.594703) (width 0.4) (layer "B.Cu") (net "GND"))
 (segment (start 74.7275 45.069) (end 80.493258 50.834758) (width 0.4) (layer "B.Cu") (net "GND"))
 (segment (start 83.4832 61.0363) (end 83.4832 52.289903) (width 0.4) (layer "B.Cu") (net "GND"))
 (segment (start 33.2281 51.231) (end 33.2281 48.9307) (width 0.4) (layer "B.Cu") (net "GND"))
 (segment (start 88.732 66.2851) (end 83.4832 61.0363) (width 0.4) (layer "B.Cu") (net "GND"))
 (segment (start 82.951615 50.931002) (end 83.4832 51.462587) (width 0.4) (layer "B.Cu") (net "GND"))
 (segment (start 83.4832 52.594703) (end 82.646901 53.431002) (width 0.4) (layer "B.Cu") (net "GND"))
 (segment (start 80.493258 50.834758) (end 80.493258 50.834845) (width 0.4) (layer "B.Cu") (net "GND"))
 (segment (start 97.3957 65.0334) (end 96.144 66.2851) (width 0.4) (layer "B.Cu") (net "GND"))
 (segment (start 101.593645 63.103045) (end 92.410055 63.103045) (width 0.4) (layer "F.Cu") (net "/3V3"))
 (segment (start 66.5182 62.2597) (end 87.002 62.2597) (width 0.4) (layer "F.Cu") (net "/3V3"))
 (segment (start 38.3081 28.6107) (end 35.7681 28.6107) (width 0.4) (layer "F.Cu") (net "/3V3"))
 (segment (start 87.002 62.2597) (end 89.7757 65.0334) (width 0.4) (layer "F.Cu") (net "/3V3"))
 (segment (start 103.524 65.0334) (end 101.593645 63.103045) (width 0.4) (layer "F.Cu") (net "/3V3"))
 (segment (start 104.7757 65.0334) (end 103.524 65.0334) (width 0.4) (layer "F.Cu") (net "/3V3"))
 (segment (start 56.4395 52.181) (end 66.5182 62.2597) (width 0.4) (layer "F.Cu") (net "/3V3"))
 (segment (start 90.4797 65.0334) (end 89.7757 65.0334) (width 0.4) (layer "F.Cu") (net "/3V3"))
 (segment (start 92.410055 63.103045) (end 90.4797 65.0334) (width 0.4) (layer "F.Cu") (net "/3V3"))
 (segment (start 56.4395 52.181) (end 55.1695 50.911) (width 0.4) (layer "B.Cu") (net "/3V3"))
 (segment (start 55.1695 50.911) (end 53.3474 50.911) (width 0.4) (layer "B.Cu") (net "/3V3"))
 (segment (start 38.3081 35.8717) (end 38.3081 28.6107) (width 0.4) (layer "B.Cu") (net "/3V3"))
 (segment (start 53.3474 50.911) (end 38.3081 35.8717) (width 0.4) (layer "B.Cu") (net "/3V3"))
 (segment (start 45.927245 31.149845) (end 43.3881 28.6107) (width 0.4) (layer "F.Cu") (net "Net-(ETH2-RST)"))
 (segment (start 81.4238 32.4401) (end 80.133545 31.149845) (width 0.4) (layer "F.Cu") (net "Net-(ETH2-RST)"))
 (segment (start 80.133545 31.149845) (end 45.927245 31.149845) (width 0.4) (layer "F.Cu") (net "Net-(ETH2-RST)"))
 (via (at 81.4238 32.4401) (size 0.6) (drill 0.3) (layers "F.Cu" "B.Cu") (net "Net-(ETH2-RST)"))
 (segment (start 80.5695 45.831) (end 81.8395 47.101) (width 0.4) (layer "B.Cu") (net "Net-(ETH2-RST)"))
 (segment (start 81.4238 32.4401) (end 80.5695 33.2944) (width 0.4) (layer "B.Cu") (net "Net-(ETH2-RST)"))
 (segment (start 80.5695 33.2944) (end 80.5695 45.831) (width 0.4) (layer "B.Cu") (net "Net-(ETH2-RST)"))
 (segment (start 53.3691 38.211) (end 45.9281 30.77) (width 0.4) (layer "B.Cu") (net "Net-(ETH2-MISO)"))
 (segment (start 57.0169 38.211) (end 53.3691 38.211) (width 0.4) (layer "B.Cu") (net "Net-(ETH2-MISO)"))
 (segment (start 57.7745 43.226) (end 57.7745 38.9686) (width 0.4) (layer "B.Cu") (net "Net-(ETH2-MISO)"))
 (segment (start 45.9281 30.77) (end 45.9281 28.6107) (width 0.4) (layer "B.Cu") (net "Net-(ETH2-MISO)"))
 (segment (start 57.7745 38.9686) (end 57.0169 38.211) (width 0.4) (layer "B.Cu") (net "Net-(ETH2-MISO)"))
 (segment (start 56.4395 44.561) (end 57.7745 43.226) (width 0.4) (layer "B.Cu") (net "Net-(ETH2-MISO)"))
 (segment (start 38.3081 48.9307) (end 41.4078 45.831) (width 0.4) (layer "F.Cu") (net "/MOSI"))
 (segment (start 41.4078 45.831) (end 55.1695 45.831) (width 0.4) (layer "F.Cu") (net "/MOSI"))
 (segment (start 55.1695 45.831) (end 56.4395 47.101) (width 0.4) (layer "F.Cu") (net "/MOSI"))
 (segment (start 55.1695 43.291) (end 42.4657 43.291) (width 0.4) (layer "F.Cu") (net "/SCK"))
 (segment (start 56.4395 42.021) (end 55.1695 43.291) (width 0.4) (layer "F.Cu") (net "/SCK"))
 (segment (start 42.4657 43.291) (end 41.3706 44.3861) (width 0.4) (layer "F.Cu") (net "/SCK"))
 (via (at 41.3706 44.3861) (size 0.6) (drill 0.3) (layers "F.Cu" "B.Cu") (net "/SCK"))
 (segment (start 41.3706 44.3861) (end 40.8481 44.9086) (width 0.4) (layer "B.Cu") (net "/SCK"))
 (segment (start 40.8481 44.9086) (end 40.8481 48.9307) (width 0.4) (layer "B.Cu") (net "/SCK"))
 (segment (start 55.1695 50.911) (end 45.3684 50.911) (width 0.4) (layer "F.Cu") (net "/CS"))
 (segment (start 56.4395 49.641) (end 55.1695 50.911) (width 0.4) (layer "F.Cu") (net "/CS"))
 (segment (start 45.3684 50.911) (end 43.3881 48.9307) (width 0.4) (layer "F.Cu") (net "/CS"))
 (segment (start 46.4878 48.371) (end 45.9281 48.9307) (width 0.4) (layer "F.Cu") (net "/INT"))
 (segment (start 54.7961 48.371) (end 54.9828 48.1843) (width 0.4) (layer "F.Cu") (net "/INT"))
 (segment (start 54.7961 48.371) (end 46.4878 48.371) (width 0.4) (layer "F.Cu") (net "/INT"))
 (via (at 54.9828 48.1843) (size 0.6) (drill 0.3) (layers "F.Cu" "B.Cu") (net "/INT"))
 (segment (start 56.4395 39.481) (end 55.1866 40.7339) (width 0.4) (layer "B.Cu") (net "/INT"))
 (segment (start 55.1866 47.9805) (end 54.9828 48.1843) (width 0.4) (layer "B.Cu") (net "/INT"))
 (segment (start 55.1866 40.7339) (end 55.1866 47.9805) (width 0.4) (layer "B.Cu") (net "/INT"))
 (segment (start 92.3157 65.0334) (end 92.3157 49.9572) (width 0.4) (layer "B.Cu") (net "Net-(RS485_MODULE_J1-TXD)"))
 (segment (start 92.3157 49.9572) (end 81.8395 39.481) (width 0.4) (layer "B.Cu") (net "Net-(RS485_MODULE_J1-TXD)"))
 (segment (start 94.8557 65.0334) (end 94.8557 49.9572) (width 0.4) (layer "B.Cu") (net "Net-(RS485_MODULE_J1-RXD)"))
 (segment (start 94.8557 49.9572) (end 81.8395 36.941) (width 0.4) (layer "B.Cu") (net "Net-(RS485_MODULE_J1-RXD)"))
 (segment (start 103.4905 45.831) (end 80.5695 45.831) (width 0.4) (layer "F.Cu") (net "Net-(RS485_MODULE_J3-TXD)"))
 (segment (start 80.5695 45.831) (end 79.2995 44.561) (width 0.4) (layer "F.Cu") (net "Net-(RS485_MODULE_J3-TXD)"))
 (segment (start 103.4905 45.831) (end 105.2302 47.5707) (width 0.4) (layer "F.Cu") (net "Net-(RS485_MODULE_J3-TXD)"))
 (via (at 105.2302 47.5707) (size 0.6) (drill 0.3) (layers "F.Cu" "B.Cu") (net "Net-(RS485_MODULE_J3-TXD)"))
 (segment (start 107.3157 49.6562) (end 105.2302 47.5707) (width 0.4) (layer "B.Cu") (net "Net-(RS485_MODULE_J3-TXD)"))
 (segment (start 107.3157 65.0334) (end 107.3157 49.6562) (width 0.4) (layer "B.Cu") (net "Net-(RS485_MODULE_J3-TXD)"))
 (segment (start 80.5695 48.371) (end 79.2995 47.101) (width 0.4) (layer "F.Cu") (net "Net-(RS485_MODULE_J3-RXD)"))
 (segment (start 106.452145 48.371045) (end 106.4521 48.371) (width 0.4) (layer "F.Cu") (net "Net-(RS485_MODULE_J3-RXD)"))
 (segment (start 110.846258 48.371045) (end 106.452145 48.371045) (width 0.4) (layer "F.Cu") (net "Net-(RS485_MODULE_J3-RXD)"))
 (segment (start 106.4521 48.371) (end 80.5695 48.371) (width 0.4) (layer "F.Cu") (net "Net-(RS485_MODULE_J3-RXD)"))
 (via (at 110.846258 48.371045) (size 0.6) (drill 0.3) (layers "F.Cu" "B.Cu") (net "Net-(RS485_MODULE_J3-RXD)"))
 (segment (start 109.8557 51.7746) (end 109.8557 65.0334) (width 0.4) (layer "B.Cu") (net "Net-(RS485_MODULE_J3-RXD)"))
 (segment (start 110.846258 50.784042) (end 109.8557 51.7746) (width 0.4) (layer "B.Cu") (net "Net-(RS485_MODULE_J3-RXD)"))
 (segment (start 110.846258 48.371045) (end 110.846258 50.784042) (width 0.4) (layer "B.Cu") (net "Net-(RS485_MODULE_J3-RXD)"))
 (segment (start 61.2655 35.925) (end 63.8055 35.925) (width 0.4) (layer "F.Cu") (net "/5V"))
 (segment (start 64.237258 37.1267) (end 64.2452 37.1267) (width 0.4) (layer "B.Cu") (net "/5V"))
 (segment (start 63.8055 35.925) (end 64.237258 36.356758) (width 0.4) (layer "B.Cu") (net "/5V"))
 (segment (start 64.2452 37.1267) (end 79.2995 52.181) (width 0.4) (layer "B.Cu") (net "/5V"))
 (segment (start 64.237258 36.356758) (end 64.237258 37.1267) (width 0.4) (layer "B.Cu") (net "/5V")))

